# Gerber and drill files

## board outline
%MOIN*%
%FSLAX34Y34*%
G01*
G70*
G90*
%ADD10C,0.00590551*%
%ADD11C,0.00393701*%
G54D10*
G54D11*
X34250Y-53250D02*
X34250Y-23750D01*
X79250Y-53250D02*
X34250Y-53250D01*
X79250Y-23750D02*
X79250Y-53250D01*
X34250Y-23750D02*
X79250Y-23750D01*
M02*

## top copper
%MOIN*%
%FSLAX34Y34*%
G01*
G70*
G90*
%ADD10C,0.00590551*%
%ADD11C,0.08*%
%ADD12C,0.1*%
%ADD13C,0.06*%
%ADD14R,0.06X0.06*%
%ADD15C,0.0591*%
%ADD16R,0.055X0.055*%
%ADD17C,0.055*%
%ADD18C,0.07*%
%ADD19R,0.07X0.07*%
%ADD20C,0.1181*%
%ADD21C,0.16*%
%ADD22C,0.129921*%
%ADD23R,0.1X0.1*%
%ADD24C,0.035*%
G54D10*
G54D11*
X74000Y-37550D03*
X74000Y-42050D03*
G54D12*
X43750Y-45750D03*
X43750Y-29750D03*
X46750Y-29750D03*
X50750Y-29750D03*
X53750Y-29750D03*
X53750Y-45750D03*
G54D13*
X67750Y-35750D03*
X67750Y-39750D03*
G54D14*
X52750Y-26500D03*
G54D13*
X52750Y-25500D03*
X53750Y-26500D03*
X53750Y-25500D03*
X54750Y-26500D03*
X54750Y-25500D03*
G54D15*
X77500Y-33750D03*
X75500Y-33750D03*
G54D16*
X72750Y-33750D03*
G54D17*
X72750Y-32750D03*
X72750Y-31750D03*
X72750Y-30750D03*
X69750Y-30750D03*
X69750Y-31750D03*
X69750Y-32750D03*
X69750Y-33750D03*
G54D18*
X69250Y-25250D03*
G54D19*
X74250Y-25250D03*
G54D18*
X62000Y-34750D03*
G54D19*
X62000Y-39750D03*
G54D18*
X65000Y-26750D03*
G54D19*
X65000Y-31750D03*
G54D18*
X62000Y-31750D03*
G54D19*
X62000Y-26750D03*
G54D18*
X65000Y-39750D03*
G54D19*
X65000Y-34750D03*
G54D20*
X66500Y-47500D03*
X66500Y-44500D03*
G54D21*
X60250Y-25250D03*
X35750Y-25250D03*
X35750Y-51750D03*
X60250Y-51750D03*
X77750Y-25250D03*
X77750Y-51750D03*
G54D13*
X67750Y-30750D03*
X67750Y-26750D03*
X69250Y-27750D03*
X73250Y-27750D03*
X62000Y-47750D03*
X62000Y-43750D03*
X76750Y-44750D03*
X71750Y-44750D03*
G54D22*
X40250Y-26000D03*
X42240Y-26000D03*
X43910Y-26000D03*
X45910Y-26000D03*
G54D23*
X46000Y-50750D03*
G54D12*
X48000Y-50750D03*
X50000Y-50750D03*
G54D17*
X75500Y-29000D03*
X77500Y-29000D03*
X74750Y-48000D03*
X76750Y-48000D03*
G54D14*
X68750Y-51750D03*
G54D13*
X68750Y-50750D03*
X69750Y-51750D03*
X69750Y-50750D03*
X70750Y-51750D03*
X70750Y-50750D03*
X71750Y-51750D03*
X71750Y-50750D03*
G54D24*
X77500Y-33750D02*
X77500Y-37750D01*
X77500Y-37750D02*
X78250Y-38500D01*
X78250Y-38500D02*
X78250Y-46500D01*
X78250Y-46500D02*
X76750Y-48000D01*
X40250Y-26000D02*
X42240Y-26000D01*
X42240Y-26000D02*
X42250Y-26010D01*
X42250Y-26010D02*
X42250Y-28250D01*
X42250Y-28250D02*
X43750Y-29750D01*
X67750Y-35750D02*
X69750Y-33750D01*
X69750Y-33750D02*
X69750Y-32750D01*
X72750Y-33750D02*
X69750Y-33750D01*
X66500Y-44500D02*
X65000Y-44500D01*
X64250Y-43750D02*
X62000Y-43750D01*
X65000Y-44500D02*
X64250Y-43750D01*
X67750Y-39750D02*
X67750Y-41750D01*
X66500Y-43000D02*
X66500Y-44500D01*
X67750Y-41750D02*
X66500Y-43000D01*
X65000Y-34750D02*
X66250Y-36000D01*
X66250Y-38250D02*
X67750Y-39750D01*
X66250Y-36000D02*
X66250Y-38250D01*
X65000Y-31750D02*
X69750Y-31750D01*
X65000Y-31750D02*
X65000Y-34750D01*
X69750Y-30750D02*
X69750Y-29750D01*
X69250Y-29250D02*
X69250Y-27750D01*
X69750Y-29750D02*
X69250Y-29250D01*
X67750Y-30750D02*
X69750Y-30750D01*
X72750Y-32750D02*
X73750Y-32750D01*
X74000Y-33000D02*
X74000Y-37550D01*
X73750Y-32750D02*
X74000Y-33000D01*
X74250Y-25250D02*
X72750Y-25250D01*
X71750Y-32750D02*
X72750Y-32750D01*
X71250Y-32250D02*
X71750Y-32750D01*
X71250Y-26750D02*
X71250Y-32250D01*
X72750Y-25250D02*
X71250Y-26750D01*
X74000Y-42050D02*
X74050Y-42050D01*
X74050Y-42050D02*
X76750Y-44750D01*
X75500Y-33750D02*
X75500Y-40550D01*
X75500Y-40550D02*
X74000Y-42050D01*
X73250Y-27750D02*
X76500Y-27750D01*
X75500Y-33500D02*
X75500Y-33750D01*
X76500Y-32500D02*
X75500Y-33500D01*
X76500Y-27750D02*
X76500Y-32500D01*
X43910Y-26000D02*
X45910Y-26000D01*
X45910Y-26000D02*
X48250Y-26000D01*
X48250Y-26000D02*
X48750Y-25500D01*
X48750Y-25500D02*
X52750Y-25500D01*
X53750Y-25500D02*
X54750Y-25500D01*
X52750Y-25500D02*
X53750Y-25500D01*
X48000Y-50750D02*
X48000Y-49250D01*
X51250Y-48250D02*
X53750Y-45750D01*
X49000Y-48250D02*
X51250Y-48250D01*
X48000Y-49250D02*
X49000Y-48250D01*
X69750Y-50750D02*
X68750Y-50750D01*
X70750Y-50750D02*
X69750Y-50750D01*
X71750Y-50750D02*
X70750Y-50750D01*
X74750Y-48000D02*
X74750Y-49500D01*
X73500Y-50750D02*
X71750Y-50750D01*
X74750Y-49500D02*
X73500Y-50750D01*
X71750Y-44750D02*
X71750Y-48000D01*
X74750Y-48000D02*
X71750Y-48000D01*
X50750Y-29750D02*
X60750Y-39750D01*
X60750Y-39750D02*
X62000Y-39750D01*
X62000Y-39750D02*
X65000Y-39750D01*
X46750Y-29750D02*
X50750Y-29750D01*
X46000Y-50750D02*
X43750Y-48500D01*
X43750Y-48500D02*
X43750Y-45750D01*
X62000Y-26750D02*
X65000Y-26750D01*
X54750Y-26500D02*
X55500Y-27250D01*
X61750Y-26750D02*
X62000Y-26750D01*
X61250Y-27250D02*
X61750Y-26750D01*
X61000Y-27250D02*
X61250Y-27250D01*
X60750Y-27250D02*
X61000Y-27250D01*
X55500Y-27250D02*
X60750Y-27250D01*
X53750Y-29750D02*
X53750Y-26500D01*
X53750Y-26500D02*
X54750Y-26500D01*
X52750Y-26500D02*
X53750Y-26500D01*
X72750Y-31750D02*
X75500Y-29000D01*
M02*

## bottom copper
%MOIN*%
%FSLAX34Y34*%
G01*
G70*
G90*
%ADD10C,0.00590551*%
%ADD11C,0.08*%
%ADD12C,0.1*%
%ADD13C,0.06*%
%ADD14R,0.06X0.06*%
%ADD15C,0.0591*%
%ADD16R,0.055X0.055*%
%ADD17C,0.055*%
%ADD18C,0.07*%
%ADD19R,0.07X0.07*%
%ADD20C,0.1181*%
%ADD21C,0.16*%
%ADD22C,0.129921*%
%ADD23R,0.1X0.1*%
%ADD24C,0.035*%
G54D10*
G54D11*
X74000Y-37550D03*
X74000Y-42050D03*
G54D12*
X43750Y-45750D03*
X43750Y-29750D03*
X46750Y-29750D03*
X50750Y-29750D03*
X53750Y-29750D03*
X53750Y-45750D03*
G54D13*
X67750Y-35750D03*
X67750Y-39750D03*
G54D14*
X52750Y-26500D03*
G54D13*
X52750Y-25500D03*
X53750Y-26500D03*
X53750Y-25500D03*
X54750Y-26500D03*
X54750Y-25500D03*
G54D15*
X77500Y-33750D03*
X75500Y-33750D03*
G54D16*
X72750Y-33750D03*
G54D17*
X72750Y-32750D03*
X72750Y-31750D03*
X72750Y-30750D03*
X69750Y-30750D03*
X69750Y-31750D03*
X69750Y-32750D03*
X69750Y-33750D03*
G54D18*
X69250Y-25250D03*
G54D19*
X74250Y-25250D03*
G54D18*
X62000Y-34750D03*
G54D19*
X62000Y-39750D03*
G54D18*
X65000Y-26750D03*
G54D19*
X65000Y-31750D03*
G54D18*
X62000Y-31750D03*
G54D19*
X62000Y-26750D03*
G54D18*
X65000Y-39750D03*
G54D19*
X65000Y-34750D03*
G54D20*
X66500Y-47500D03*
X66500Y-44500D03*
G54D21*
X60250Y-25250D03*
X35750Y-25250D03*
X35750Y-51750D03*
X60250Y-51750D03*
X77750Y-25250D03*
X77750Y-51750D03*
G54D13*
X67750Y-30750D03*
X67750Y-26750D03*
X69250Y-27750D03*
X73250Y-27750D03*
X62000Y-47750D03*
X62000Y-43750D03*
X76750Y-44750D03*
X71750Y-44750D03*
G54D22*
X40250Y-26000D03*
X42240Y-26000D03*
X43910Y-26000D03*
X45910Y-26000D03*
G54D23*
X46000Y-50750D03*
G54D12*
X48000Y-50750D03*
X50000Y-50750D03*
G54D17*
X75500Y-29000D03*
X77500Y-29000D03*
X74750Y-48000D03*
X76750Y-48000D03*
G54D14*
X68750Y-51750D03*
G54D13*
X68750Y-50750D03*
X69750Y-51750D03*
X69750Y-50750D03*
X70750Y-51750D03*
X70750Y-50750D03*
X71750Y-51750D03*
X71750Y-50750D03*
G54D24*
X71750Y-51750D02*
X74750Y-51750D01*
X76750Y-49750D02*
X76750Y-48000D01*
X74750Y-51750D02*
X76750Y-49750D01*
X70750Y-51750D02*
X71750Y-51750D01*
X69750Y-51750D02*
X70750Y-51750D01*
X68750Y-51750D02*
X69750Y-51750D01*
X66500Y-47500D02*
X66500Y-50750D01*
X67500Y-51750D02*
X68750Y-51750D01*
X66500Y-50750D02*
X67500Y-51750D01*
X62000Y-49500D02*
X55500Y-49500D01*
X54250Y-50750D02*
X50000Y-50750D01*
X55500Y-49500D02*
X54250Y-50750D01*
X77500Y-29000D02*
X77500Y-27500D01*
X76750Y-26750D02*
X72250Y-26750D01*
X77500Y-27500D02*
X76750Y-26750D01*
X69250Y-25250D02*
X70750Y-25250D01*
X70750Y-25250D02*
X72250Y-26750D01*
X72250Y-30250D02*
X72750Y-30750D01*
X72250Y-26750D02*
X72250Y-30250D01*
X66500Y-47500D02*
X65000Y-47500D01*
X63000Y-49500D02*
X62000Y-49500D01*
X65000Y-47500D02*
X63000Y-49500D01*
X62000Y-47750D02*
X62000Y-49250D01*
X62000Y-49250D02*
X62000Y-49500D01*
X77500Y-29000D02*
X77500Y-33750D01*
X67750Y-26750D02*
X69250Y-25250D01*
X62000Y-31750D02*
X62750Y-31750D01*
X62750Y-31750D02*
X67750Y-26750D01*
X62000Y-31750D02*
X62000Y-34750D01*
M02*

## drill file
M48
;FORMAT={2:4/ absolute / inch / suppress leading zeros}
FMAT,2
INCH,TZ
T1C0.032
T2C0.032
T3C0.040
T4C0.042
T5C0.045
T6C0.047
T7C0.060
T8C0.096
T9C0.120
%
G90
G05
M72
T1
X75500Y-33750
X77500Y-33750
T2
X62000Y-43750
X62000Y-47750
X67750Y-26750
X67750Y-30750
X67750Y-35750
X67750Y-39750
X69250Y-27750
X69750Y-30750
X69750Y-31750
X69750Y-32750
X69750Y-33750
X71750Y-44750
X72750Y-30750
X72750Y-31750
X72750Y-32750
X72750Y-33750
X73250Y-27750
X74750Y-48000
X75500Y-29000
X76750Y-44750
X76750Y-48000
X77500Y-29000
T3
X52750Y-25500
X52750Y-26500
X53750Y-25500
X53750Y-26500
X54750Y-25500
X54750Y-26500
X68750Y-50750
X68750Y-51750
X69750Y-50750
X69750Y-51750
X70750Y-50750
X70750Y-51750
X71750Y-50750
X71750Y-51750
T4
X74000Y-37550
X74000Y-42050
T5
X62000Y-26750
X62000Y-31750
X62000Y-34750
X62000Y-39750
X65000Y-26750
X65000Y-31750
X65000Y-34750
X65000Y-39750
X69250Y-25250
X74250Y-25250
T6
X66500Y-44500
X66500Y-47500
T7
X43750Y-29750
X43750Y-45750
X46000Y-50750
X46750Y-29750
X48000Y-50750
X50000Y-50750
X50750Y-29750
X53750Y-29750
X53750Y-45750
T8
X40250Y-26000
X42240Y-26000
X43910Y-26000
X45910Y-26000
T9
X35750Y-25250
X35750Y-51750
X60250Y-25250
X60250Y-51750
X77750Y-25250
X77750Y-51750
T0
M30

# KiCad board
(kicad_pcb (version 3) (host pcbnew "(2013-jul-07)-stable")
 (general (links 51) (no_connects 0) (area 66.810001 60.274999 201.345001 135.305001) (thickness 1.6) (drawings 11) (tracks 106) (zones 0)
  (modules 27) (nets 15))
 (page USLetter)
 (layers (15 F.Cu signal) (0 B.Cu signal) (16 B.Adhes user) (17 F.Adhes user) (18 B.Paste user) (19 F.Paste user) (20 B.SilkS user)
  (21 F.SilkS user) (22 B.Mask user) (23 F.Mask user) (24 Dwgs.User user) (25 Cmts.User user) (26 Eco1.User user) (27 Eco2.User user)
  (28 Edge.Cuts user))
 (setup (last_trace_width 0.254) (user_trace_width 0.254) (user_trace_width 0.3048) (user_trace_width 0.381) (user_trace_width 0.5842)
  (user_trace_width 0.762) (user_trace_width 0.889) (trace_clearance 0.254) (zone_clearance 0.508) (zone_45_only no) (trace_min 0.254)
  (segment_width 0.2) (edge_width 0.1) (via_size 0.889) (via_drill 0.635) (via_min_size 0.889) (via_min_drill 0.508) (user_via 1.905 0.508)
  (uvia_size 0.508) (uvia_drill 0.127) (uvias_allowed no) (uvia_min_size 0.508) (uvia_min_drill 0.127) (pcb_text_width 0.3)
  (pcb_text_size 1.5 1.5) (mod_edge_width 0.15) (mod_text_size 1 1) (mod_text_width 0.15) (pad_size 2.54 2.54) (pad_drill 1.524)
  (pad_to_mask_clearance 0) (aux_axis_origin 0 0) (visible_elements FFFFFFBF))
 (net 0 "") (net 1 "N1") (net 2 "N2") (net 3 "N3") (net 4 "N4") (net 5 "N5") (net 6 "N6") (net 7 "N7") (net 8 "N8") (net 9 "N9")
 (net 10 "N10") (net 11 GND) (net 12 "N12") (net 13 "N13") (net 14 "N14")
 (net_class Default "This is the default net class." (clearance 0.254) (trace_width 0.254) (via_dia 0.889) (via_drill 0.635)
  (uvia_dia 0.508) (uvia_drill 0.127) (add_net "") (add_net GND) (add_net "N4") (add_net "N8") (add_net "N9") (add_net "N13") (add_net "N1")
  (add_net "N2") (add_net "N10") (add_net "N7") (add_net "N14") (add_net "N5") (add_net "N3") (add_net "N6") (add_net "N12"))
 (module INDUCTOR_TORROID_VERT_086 (layer F.Cu) (at 187.96 100.965)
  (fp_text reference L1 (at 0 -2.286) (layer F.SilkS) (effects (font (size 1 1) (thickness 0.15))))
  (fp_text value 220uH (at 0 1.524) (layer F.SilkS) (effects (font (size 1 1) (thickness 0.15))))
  (pad 1 thru_hole circle (at 0 -5.588) (size 2.032 2.032) (drill 1.0668) (layers *.Cu *.Mask F.SilkS) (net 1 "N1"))
  (pad 2 thru_hole circle (at 0 5.842) (size 2.032 2.032) (drill 1.0668) (layers *.Cu *.Mask F.SilkS) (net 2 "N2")))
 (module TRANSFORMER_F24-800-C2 (layer F.Cu) (at 123.825 75.565)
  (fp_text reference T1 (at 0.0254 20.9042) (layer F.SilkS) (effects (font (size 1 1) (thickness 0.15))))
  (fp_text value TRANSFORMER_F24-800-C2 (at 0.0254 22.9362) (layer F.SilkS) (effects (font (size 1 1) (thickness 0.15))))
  (pad 1 thru_hole circle (at -12.7 40.64) (size 2.54 2.54) (drill 1.524) (layers *.Cu *.Mask F.SilkS) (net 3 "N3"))
  (pad 5 thru_hole circle (at -12.7 0) (size 2.54 2.54) (drill 1.524) (layers *.Cu *.Mask F.SilkS) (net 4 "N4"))
  (pad 6 thru_hole circle (at -5.08 0) (size 2.54 2.54) (drill 1.524) (layers *.Cu *.Mask F.SilkS) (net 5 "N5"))
  (pad 7 thru_hole circle (at 5.08 0) (size 2.54 2.54) (drill 1.524) (layers *.Cu *.Mask F.SilkS) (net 5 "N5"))
  (pad 8 thru_hole circle (at 12.7 0) (size 2.54 2.54) (drill 1.524) (layers *.Cu *.Mask F.SilkS) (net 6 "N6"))
  (pad 4 thru_hole circle (at 12.7 40.64) (size 2.54 2.54) (drill 1.524) (layers *.Cu *.Mask F.SilkS) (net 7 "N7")))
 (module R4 (layer F.Cu) (at 172.085 95.885 270) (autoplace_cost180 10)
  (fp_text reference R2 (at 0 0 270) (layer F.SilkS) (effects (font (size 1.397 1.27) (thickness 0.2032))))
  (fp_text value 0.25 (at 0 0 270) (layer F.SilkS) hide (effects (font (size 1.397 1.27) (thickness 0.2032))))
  (pad 1 thru_hole circle (at -5.08 0 270) (size 1.524 1.524) (drill 0.8128) (layers *.Cu *.Mask F.SilkS) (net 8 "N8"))
  (pad 2 thru_hole circle (at 5.08 0 270) (size 1.524 1.524) (drill 0.8128) (layers *.Cu *.Mask F.SilkS) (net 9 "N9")))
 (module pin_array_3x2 (layer F.Cu) (at 136.525 66.04)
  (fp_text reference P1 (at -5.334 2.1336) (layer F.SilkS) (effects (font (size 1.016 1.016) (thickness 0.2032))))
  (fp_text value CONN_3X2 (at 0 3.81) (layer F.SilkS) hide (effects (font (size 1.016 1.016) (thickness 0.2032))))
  (pad 1 thru_hole rect (at -2.54 1.27) (size 1.524 1.524) (drill 1.016) (layers *.Cu *.Mask F.SilkS) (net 6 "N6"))
  (pad 2 thru_hole circle (at -2.54 -1.27) (size 1.524 1.524) (drill 1.016) (layers *.Cu *.Mask F.SilkS) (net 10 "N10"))
  (pad 3 thru_hole circle (at 0 1.27) (size 1.524 1.524) (drill 1.016) (layers *.Cu *.Mask F.SilkS) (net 6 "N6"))
  (pad 4 thru_hole circle (at 0 -1.27) (size 1.524 1.524) (drill 1.016) (layers *.Cu *.Mask F.SilkS) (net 10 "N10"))
  (pad 5 thru_hole circle (at 2.54 1.27) (size 1.524 1.524) (drill 1.016) (layers *.Cu *.Mask F.SilkS) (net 6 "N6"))
  (pad 6 thru_hole circle (at 2.54 -1.27) (size 1.524 1.524) (drill 1.016) (layers *.Cu *.Mask F.SilkS) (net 10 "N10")))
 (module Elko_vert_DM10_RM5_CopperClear (layer F.Cu) (at 194.31 85.725)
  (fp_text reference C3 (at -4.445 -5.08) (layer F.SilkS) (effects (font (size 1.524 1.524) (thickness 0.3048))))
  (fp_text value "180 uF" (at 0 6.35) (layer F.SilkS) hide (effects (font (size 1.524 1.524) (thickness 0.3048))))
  (pad 2 thru_hole circle (at 2.54 0) (size 1.50114 1.50114) (drill 0.8001) (layers *.Cu *.Mask F.SilkS) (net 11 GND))
  (pad 1 thru_hole circle (at -2.54 0) (size 1.50114 1.50114) (drill 0.8001) (layers *.Cu *.Mask F.SilkS) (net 2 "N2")))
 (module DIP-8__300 (layer F.Cu) (at 180.975 81.915 90)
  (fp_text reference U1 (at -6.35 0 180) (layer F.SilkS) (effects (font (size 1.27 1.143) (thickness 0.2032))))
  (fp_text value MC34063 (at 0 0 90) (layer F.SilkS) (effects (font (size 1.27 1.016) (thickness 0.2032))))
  (pad 1 thru_hole rect (at -3.81 3.81 90) (size 1.397 1.397) (drill 0.8128) (layers *.Cu *.Mask F.SilkS) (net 8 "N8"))
  (pad 2 thru_hole circle (at -1.27 3.81 90) (size 1.397 1.397) (drill 0.8128) (layers *.Cu *.Mask F.SilkS) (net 1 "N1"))
  (pad 3 thru_hole circle (at 1.27 3.81 90) (size 1.397 1.397) (drill 0.8128) (layers *.Cu *.Mask F.SilkS) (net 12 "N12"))
  (pad 4 thru_hole circle (at 3.81 3.81 90) (size 1.397 1.397) (drill 0.8128) (layers *.Cu *.Mask F.SilkS) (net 11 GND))
  (pad 5 thru_hole circle (at 3.81 -3.81 90) (size 1.397 1.397) (drill 0.8128) (layers *.Cu *.Mask F.SilkS) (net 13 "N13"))
  (pad 6 thru_hole circle (at 1.27 -3.81 90) (size 1.397 1.397) (drill 0.8128) (layers *.Cu *.Mask F.SilkS) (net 9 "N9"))
  (pad 7 thru_hole circle (at -1.27 -3.81 90) (size 1.397 1.397) (drill 0.8128) (layers *.Cu *.Mask F.SilkS) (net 8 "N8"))
  (pad 8 thru_hole circle (at -3.81 -3.81 90) (size 1.397 1.397) (drill 0.8128) (layers *.Cu *.Mask F.SilkS) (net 8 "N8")))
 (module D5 (layer F.Cu) (at 182.245 64.135)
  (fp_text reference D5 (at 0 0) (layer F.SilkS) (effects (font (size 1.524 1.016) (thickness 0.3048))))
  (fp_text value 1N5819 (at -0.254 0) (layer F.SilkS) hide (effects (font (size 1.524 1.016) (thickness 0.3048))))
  (pad 1 thru_hole circle (at -6.35 0) (size 1.778 1.778) (drill 1.143) (layers *.Cu *.Mask F.SilkS) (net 11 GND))
  (pad 2 thru_hole rect (at 6.35 0) (size 1.778 1.778) (drill 1.143) (layers *.Cu *.Mask F.SilkS) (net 1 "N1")))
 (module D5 (layer F.Cu) (at 157.48 94.615 270)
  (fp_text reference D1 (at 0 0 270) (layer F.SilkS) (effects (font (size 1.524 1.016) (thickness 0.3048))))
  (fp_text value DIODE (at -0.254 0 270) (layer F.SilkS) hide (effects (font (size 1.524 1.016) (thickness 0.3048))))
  (pad 1 thru_hole circle (at -6.35 0 270) (size 1.778 1.778) (drill 1.143) (layers *.Cu *.Mask F.SilkS) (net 11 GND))
  (pad 2 thru_hole rect (at 6.35 0 270) (size 1.778 1.778) (drill 1.143) (layers *.Cu *.Mask F.SilkS) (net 5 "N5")))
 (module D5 (layer F.Cu) (at 165.1 74.295 270)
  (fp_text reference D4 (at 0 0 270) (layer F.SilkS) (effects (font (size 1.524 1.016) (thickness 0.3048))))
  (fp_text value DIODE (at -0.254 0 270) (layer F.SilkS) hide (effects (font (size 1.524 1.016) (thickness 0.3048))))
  (pad 1 thru_hole circle (at -6.35 0 270) (size 1.778 1.778) (drill 1.143) (layers *.Cu *.Mask F.SilkS) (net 6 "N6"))
  (pad 2 thru_hole rect (at 6.35 0 270) (size 1.778 1.778) (drill 1.143) (layers *.Cu *.Mask F.SilkS) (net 9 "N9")))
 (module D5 (layer F.Cu) (at 157.48 74.295 90)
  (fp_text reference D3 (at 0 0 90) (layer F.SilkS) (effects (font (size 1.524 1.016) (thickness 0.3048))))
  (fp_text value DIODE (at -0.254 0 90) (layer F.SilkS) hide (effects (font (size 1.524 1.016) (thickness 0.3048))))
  (pad 1 thru_hole circle (at -6.35 0 90) (size 1.778 1.778) (drill 1.143) (layers *.Cu *.Mask F.SilkS) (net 11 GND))
  (pad 2 thru_hole rect (at 6.35 0 90) (size 1.778 1.778) (drill 1.143) (layers *.Cu *.Mask F.SilkS) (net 6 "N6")))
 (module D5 (layer F.Cu) (at 165.1 94.615 90)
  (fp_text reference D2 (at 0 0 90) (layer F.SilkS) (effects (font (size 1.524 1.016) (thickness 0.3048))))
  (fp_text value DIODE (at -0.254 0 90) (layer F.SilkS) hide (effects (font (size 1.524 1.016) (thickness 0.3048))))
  (pad 1 thru_hole circle (at -6.35 0 90) (size 1.778 1.778) (drill 1.143) (layers *.Cu *.Mask F.SilkS) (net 5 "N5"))
  (pad 2 thru_hole rect (at 6.35 0 90) (size 1.778 1.778) (drill 1.143) (layers *.Cu *.Mask F.SilkS) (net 9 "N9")))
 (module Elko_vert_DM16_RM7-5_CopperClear (layer F.Cu) (at 168.91 116.84 270)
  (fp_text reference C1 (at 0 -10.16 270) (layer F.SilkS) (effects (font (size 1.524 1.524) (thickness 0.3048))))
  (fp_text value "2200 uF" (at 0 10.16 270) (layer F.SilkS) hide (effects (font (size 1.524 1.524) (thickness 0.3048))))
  (pad 2 thru_hole circle (at 3.81 0 270) (size 2.99974 2.99974) (drill 1.19888) (layers *.Cu *.Mask F.SilkS) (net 11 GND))
  (pad 1 thru_hole circle (at -3.81 0 270) (size 2.99974 2.99974) (drill 1.19888) (layers *.Cu *.Mask F.SilkS) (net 9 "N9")))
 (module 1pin (layer F.Cu) (at 153.035 64.135)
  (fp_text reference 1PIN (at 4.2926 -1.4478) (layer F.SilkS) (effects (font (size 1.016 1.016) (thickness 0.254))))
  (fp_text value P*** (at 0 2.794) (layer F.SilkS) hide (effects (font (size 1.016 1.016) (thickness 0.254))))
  (pad 1 thru_hole circle (at 0 0) (size 4.064 4.064) (drill 3.048) (layers *.Cu *.Mask F.SilkS)))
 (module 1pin (layer F.Cu) (at 90.805 64.135)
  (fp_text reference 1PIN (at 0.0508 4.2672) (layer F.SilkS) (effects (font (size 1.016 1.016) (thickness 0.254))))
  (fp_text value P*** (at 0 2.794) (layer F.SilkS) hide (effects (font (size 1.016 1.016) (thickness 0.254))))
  (pad 1 thru_hole circle (at 0 0) (size 4.064 4.064) (drill 3.048) (layers *.Cu *.Mask F.SilkS)))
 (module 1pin (layer F.Cu) (at 90.805 131.445)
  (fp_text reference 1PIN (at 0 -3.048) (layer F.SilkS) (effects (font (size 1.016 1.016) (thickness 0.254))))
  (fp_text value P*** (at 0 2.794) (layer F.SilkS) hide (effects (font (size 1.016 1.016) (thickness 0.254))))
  (pad 1 thru_hole circle (at 0 0) (size 4.064 4.064) (drill 3.048) (layers *.Cu *.Mask F.SilkS)))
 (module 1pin (layer F.Cu) (at 153.035 131.445)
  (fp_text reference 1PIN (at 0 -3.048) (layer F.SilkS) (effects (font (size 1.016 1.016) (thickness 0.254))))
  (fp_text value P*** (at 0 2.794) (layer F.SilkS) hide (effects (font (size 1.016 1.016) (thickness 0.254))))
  (pad 1 thru_hole circle (at 0 0) (size 4.064 4.064) (drill 3.048) (layers *.Cu *.Mask F.SilkS)))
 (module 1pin (layer F.Cu) (at 197.485 64.135)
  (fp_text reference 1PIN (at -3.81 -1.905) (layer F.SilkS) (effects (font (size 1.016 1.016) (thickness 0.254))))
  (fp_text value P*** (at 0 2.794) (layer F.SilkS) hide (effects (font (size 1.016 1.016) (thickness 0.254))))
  (pad 1 thru_hole circle (at 0 0) (size 4.064 4.064) (drill 3.048) (layers *.Cu *.Mask F.SilkS)))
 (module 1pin (layer F.Cu) (at 197.485 131.445)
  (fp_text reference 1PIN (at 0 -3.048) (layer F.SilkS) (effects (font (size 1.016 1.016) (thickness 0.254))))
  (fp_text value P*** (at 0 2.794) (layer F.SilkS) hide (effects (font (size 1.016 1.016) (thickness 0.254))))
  (pad 1 thru_hole circle (at 0 0) (size 4.064 4.064) (drill 3.048) (layers *.Cu *.Mask F.SilkS)))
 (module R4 (layer F.Cu) (at 172.085 73.025 90) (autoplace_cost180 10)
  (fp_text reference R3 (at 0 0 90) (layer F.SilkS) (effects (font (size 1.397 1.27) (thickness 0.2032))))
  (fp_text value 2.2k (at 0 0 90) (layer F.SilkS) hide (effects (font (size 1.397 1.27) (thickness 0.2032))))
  (pad 1 thru_hole circle (at -5.08 0 90) (size 1.524 1.524) (drill 0.8128) (layers *.Cu *.Mask F.SilkS) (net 13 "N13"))
  (pad 2 thru_hole circle (at 5.08 0 90) (size 1.524 1.524) (drill 0.8128) (layers *.Cu *.Mask F.SilkS) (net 11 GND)))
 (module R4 (layer F.Cu) (at 180.975 70.485) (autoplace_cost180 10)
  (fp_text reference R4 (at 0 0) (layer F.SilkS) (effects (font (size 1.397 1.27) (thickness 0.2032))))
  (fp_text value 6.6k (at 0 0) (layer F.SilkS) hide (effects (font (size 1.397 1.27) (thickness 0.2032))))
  (pad 1 thru_hole circle (at -5.08 0) (size 1.524 1.524) (drill 0.8128) (layers *.Cu *.Mask F.SilkS) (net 13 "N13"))
  (pad 2 thru_hole circle (at 5.08 0) (size 1.524 1.524) (drill 0.8128) (layers *.Cu *.Mask F.SilkS) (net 2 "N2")))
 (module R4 (layer F.Cu) (at 157.48 116.205 90) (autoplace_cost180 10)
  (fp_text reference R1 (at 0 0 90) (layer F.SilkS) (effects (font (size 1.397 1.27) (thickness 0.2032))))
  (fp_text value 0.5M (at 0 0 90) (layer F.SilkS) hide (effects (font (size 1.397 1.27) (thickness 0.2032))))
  (pad 1 thru_hole circle (at -5.08 0 90) (size 1.524 1.524) (drill 0.8128) (layers *.Cu *.Mask F.SilkS) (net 11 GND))
  (pad 2 thru_hole circle (at 5.08 0 90) (size 1.524 1.524) (drill 0.8128) (layers *.Cu *.Mask F.SilkS) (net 9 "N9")))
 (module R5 (layer F.Cu) (at 188.595 113.665 180) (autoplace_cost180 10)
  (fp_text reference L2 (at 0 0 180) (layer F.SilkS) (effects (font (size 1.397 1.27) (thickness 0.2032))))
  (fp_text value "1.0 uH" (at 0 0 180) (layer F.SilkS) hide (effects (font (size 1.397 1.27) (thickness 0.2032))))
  (pad 1 thru_hole circle (at -6.35 0 180) (size 1.524 1.524) (drill 0.8128) (layers *.Cu *.Mask F.SilkS) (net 2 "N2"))
  (pad 2 thru_hole circle (at 6.35 0 180) (size 1.524 1.524) (drill 0.8128) (layers *.Cu *.Mask F.SilkS) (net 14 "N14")))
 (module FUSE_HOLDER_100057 (layer F.Cu) (at 109.855 66.04)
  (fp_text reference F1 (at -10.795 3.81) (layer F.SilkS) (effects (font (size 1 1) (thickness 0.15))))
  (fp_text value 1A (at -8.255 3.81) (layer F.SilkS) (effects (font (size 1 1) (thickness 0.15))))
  (pad 1 thru_hole circle (at -7.62 0) (size 3.3 3.3) (drill 2.44) (layers *.Cu *.Mask F.SilkS) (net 4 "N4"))
  (pad 1 thru_hole circle (at -2.5654 0) (size 3.3 3.3) (drill 2.44) (layers *.Cu *.Mask F.SilkS) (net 4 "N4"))
  (pad 2 thru_hole circle (at 1.6764 0) (size 3.3 3.3) (drill 2.44) (layers *.Cu *.Mask F.SilkS) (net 10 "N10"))
  (pad 2 thru_hole circle (at 6.7564 0) (size 3.3 3.3) (drill 2.44) (layers *.Cu *.Mask F.SilkS) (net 10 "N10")))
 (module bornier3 (layer F.Cu) (at 121.92 128.905)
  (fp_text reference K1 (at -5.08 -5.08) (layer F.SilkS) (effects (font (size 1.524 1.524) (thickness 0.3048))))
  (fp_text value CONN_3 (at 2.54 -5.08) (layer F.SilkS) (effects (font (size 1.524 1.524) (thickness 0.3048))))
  (pad 1 thru_hole rect (at -5.08 0) (size 2.54 2.54) (drill 1.524) (layers *.Cu *.Mask F.SilkS) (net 3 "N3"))
  (pad 2 thru_hole circle (at 0 0) (size 2.54 2.54) (drill 1.524) (layers *.Cu *.Mask F.SilkS) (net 7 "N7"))
  (pad 3 thru_hole circle (at 5.08 0) (size 2.54 2.54) (drill 1.524) (layers *.Cu *.Mask F.SilkS) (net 11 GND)))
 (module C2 (layer F.Cu) (at 194.31 73.66)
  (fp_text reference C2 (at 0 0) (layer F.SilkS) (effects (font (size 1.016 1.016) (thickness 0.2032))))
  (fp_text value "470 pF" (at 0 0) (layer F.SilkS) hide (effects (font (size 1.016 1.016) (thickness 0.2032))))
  (pad 1 thru_hole circle (at -2.54 0) (size 1.397 1.397) (drill 0.8128) (layers *.Cu *.Mask F.SilkS) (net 12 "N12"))
  (pad 2 thru_hole circle (at 2.54 0) (size 1.397 1.397) (drill 0.8128) (layers *.Cu *.Mask F.SilkS) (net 11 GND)))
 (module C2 (layer F.Cu) (at 192.405 121.92)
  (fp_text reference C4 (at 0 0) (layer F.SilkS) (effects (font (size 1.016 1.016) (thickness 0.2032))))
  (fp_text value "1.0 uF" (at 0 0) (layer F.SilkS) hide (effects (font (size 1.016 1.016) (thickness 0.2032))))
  (pad 1 thru_hole circle (at -2.54 0) (size 1.397 1.397) (drill 0.8128) (layers *.Cu *.Mask F.SilkS) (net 14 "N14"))
  (pad 2 thru_hole circle (at 2.54 0) (size 1.397 1.397) (drill 0.8128) (layers *.Cu *.Mask F.SilkS) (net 11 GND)))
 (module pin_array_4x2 (layer F.Cu) (at 178.435 130.175)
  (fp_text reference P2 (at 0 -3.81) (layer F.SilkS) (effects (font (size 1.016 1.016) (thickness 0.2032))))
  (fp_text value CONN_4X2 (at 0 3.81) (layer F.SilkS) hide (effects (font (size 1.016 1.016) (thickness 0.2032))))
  (pad 1 thru_hole rect (at -3.81 1.27) (size 1.524 1.524) (drill 1.016) (layers *.Cu *.Mask F.SilkS) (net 11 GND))
  (pad 2 thru_hole circle (at -3.81 -1.27) (size 1.524 1.524) (drill 1.016) (layers *.Cu *.Mask F.SilkS) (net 14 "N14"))
  (pad 3 thru_hole circle (at -1.27 1.27) (size 1.524 1.524) (drill 1.016) (layers *.Cu *.Mask F.SilkS) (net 11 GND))
  (pad 4 thru_hole circle (at -1.27 -1.27) (size 1.524 1.524) (drill 1.016) (layers *.Cu *.Mask F.SilkS) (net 14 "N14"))
  (pad 5 thru_hole circle (at 1.27 1.27) (size 1.524 1.524) (drill 1.016) (layers *.Cu *.Mask F.SilkS) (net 11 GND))
  (pad 6 thru_hole circle (at 1.27 -1.27) (size 1.524 1.524) (drill 1.016) (layers *.Cu *.Mask F.SilkS) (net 14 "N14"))
  (pad 7 thru_hole circle (at 3.81 1.27) (size 1.524 1.524) (drill 1.016) (layers *.Cu *.Mask F.SilkS) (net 11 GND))
  (pad 8 thru_hole circle (at 3.81 -1.27) (size 1.524 1.524) (drill 1.016) (layers *.Cu *.Mask F.SilkS) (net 14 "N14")))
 (gr_line (start 86.995 135.255) (end 86.995 60.325) (angle 90) (layer Edge.Cuts) (width 0.1))
 (gr_line (start 201.295 135.255) (end 86.995 135.255) (angle 90) (layer Edge.Cuts) (width 0.1))
 (gr_line (start 201.295 60.325) (end 201.295 135.255) (angle 90) (layer Edge.Cuts) (width 0.1))
 (gr_line (start 86.995 60.325) (end 201.295 60.325) (angle 90) (layer Edge.Cuts) (width 0.1))
 (segment (start 182.245 131.445) (end 189.865 131.445) (width 0.889) (layer B.Cu) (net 11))
 (segment (start 194.945 126.365) (end 194.945 121.92) (width 0.889) (layer B.Cu) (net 11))
 (segment (start 189.865 131.445) (end 194.945 126.365) (width 0.889) (layer B.Cu) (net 11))
 (segment (start 179.705 131.445) (end 182.245 131.445) (width 0.889) (layer B.Cu) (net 11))
 (segment (start 177.165 131.445) (end 179.705 131.445) (width 0.889) (layer B.Cu) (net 11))
 (segment (start 174.625 131.445) (end 177.165 131.445) (width 0.889) (layer B.Cu) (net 11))
 (segment (start 168.91 120.65) (end 168.91 128.905) (width 0.889) (layer B.Cu) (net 11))
 (segment (start 171.45 131.445) (end 174.625 131.445) (width 0.889) (layer B.Cu) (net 11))
 (segment (start 168.91 128.905) (end 171.45 131.445) (width 0.889) (layer B.Cu) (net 11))
 (segment (start 157.48 125.73) (end 140.97 125.73) (width 0.889) (layer B.Cu) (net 11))
 (segment (start 137.795 128.905) (end 127 128.905) (width 0.889) (layer B.Cu) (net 11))
 (segment (start 140.97 125.73) (end 137.795 128.905) (width 0.889) (layer B.Cu) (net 11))
 (segment (start 196.85 73.66) (end 196.85 69.85) (width 0.889) (layer B.Cu) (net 11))
 (segment (start 194.945 67.945) (end 183.515 67.945) (width 0.889) (layer B.Cu) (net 11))
 (segment (start 196.85 69.85) (end 194.945 67.945) (width 0.889) (layer B.Cu) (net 11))
 (segment (start 175.895 64.135) (end 179.705 64.135) (width 0.889) (layer B.Cu) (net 11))
 (segment (start 179.705 64.135) (end 183.515 67.945) (width 0.889) (layer B.Cu) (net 11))
 (segment (start 183.515 76.835) (end 184.785 78.105) (width 0.889) (layer B.Cu) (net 11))
 (segment (start 183.515 67.945) (end 183.515 76.835) (width 0.889) (layer B.Cu) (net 11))
 (segment (start 168.91 120.65) (end 165.1 120.65) (width 0.889) (layer B.Cu) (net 11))
 (segment (start 160.02 125.73) (end 157.48 125.73) (width 0.889) (layer B.Cu) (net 11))
 (segment (start 165.1 120.65) (end 160.02 125.73) (width 0.889) (layer B.Cu) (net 11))
 (segment (start 157.48 121.285) (end 157.48 125.095) (width 0.889) (layer B.Cu) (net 11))
 (segment (start 157.48 125.095) (end 157.48 125.73) (width 0.889) (layer B.Cu) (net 11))
 (segment (start 196.85 85.725) (end 196.85 95.885) (width 0.889) (layer F.Cu) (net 11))
 (segment (start 196.85 95.885) (end 198.755 97.79) (width 0.889) (layer F.Cu) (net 11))
 (segment (start 198.755 97.79) (end 198.755 118.11) (width 0.889) (layer F.Cu) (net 11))
 (segment (start 198.755 118.11) (end 194.945 121.92) (width 0.889) (layer F.Cu) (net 11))
 (segment (start 196.85 73.66) (end 196.85 85.725) (width 0.889) (layer B.Cu) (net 11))
 (segment (start 172.085 67.945) (end 175.895 64.135) (width 0.889) (layer B.Cu) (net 11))
 (segment (start 157.48 80.645) (end 159.385 80.645) (width 0.889) (layer B.Cu) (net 11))
 (segment (start 159.385 80.645) (end 172.085 67.945) (width 0.889) (layer B.Cu) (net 11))
 (segment (start 157.48 80.645) (end 157.48 88.265) (width 0.889) (layer B.Cu) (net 11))
 (segment (start 102.235 66.04) (end 107.2896 66.04) (width 0.889) (layer F.Cu) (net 4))
 (segment (start 107.2896 66.04) (end 107.315 66.0654) (width 0.889) (layer F.Cu) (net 4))
 (segment (start 107.315 66.0654) (end 107.315 71.755) (width 0.889) (layer F.Cu) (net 4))
 (segment (start 107.315 71.755) (end 111.125 75.565) (width 0.889) (layer F.Cu) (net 4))
 (segment (start 172.085 90.805) (end 177.165 85.725) (width 0.889) (layer F.Cu) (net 8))
 (segment (start 177.165 85.725) (end 177.165 83.185) (width 0.889) (layer F.Cu) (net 8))
 (segment (start 184.785 85.725) (end 177.165 85.725) (width 0.889) (layer F.Cu) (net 8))
 (segment (start 168.91 113.03) (end 165.1 113.03) (width 0.889) (layer F.Cu) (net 9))
 (segment (start 163.195 111.125) (end 157.48 111.125) (width 0.889) (layer F.Cu) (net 9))
 (segment (start 165.1 113.03) (end 163.195 111.125) (width 0.889) (layer F.Cu) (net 9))
 (segment (start 172.085 100.965) (end 172.085 106.045) (width 0.889) (layer F.Cu) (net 9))
 (segment (start 168.91 109.22) (end 168.91 113.03) (width 0.889) (layer F.Cu) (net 9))
 (segment (start 172.085 106.045) (end 168.91 109.22) (width 0.889) (layer F.Cu) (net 9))
 (segment (start 165.1 88.265) (end 168.275 91.44) (width 0.889) (layer F.Cu) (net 9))
 (segment (start 168.275 97.155) (end 172.085 100.965) (width 0.889) (layer F.Cu) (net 9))
 (segment (start 168.275 91.44) (end 168.275 97.155) (width 0.889) (layer F.Cu) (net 9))
 (segment (start 165.1 80.645) (end 177.165 80.645) (width 0.889) (layer F.Cu) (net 9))
 (segment (start 165.1 80.645) (end 165.1 88.265) (width 0.889) (layer F.Cu) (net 9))
 (segment (start 177.165 78.105) (end 177.165 75.565) (width 0.889) (layer F.Cu) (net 13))
 (segment (start 175.895 74.295) (end 175.895 70.485) (width 0.889) (layer F.Cu) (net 13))
 (segment (start 177.165 75.565) (end 175.895 74.295) (width 0.889) (layer F.Cu) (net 13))
 (segment (start 172.085 78.105) (end 177.165 78.105) (width 0.889) (layer F.Cu) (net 13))
 (segment (start 184.785 83.185) (end 187.325 83.185) (width 0.889) (layer F.Cu) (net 1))
 (segment (start 187.96 83.82) (end 187.96 95.377) (width 0.889) (layer F.Cu) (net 1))
 (segment (start 187.325 83.185) (end 187.96 83.82) (width 0.889) (layer F.Cu) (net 1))
 (segment (start 188.595 64.135) (end 184.785 64.135) (width 0.889) (layer F.Cu) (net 1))
 (segment (start 182.245 83.185) (end 184.785 83.185) (width 0.889) (layer F.Cu) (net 1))
 (segment (start 180.975 81.915) (end 182.245 83.185) (width 0.889) (layer F.Cu) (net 1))
 (segment (start 180.975 67.945) (end 180.975 81.915) (width 0.889) (layer F.Cu) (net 1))
 (segment (start 184.785 64.135) (end 180.975 67.945) (width 0.889) (layer F.Cu) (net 1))
 (segment (start 187.96 106.807) (end 188.087 106.807) (width 0.889) (layer F.Cu) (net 2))
 (segment (start 188.087 106.807) (end 194.945 113.665) (width 0.889) (layer F.Cu) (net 2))
 (segment (start 191.77 85.725) (end 191.77 102.997) (width 0.889) (layer F.Cu) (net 2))
 (segment (start 191.77 102.997) (end 187.96 106.807) (width 0.889) (layer F.Cu) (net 2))
 (segment (start 186.055 70.485) (end 194.31 70.485) (width 0.889) (layer F.Cu) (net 2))
 (segment (start 191.77 85.09) (end 191.77 85.725) (width 0.889) (layer F.Cu) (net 2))
 (segment (start 194.31 82.55) (end 191.77 85.09) (width 0.889) (layer F.Cu) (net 2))
 (segment (start 194.31 70.485) (end 194.31 82.55) (width 0.889) (layer F.Cu) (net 2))
 (segment (start 111.5314 66.04) (end 116.6114 66.04) (width 0.889) (layer F.Cu) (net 10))
 (segment (start 116.6114 66.04) (end 122.555 66.04) (width 0.889) (layer F.Cu) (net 10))
 (segment (start 122.555 66.04) (end 123.825 64.77) (width 0.889) (layer F.Cu) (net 10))
 (segment (start 123.825 64.77) (end 133.985 64.77) (width 0.889) (layer F.Cu) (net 10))
 (segment (start 136.525 64.77) (end 139.065 64.77) (width 0.889) (layer F.Cu) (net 10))
 (segment (start 133.985 64.77) (end 136.525 64.77) (width 0.889) (layer F.Cu) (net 10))
 (segment (start 121.92 128.905) (end 121.92 125.095) (width 0.889) (layer F.Cu) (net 7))
 (segment (start 130.175 122.555) (end 136.525 116.205) (width 0.889) (layer F.Cu) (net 7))
 (segment (start 124.46 122.555) (end 130.175 122.555) (width 0.889) (layer F.Cu) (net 7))
 (segment (start 121.92 125.095) (end 124.46 122.555) (width 0.889) (layer F.Cu) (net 7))
 (segment (start 177.165 128.905) (end 174.625 128.905) (width 0.889) (layer F.Cu) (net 14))
 (segment (start 179.705 128.905) (end 177.165 128.905) (width 0.889) (layer F.Cu) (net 14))
 (segment (start 182.245 128.905) (end 179.705 128.905) (width 0.889) (layer F.Cu) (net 14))
 (segment (start 189.865 121.92) (end 189.865 125.73) (width 0.889) (layer F.Cu) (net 14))
 (segment (start 186.69 128.905) (end 182.245 128.905) (width 0.889) (layer F.Cu) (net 14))
 (segment (start 189.865 125.73) (end 186.69 128.905) (width 0.889) (layer F.Cu) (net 14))
 (segment (start 182.245 113.665) (end 182.245 121.92) (width 0.889) (layer F.Cu) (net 14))
 (segment (start 189.865 121.92) (end 182.245 121.92) (width 0.889) (layer F.Cu) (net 14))
 (segment (start 128.905 75.565) (end 154.305 100.965) (width 0.889) (layer F.Cu) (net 5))
 (segment (start 154.305 100.965) (end 157.48 100.965) (width 0.889) (layer F.Cu) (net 5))
 (segment (start 157.48 100.965) (end 165.1 100.965) (width 0.889) (layer F.Cu) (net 5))
 (segment (start 118.745 75.565) (end 128.905 75.565) (width 0.889) (layer F.Cu) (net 5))
 (segment (start 116.84 128.905) (end 111.125 123.19) (width 0.889) (layer F.Cu) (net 3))
 (segment (start 111.125 123.19) (end 111.125 116.205) (width 0.889) (layer F.Cu) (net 3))
 (segment (start 157.48 67.945) (end 165.1 67.945) (width 0.889) (layer F.Cu) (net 6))
 (segment (start 139.065 67.31) (end 140.97 69.215) (width 0.889) (layer F.Cu) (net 6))
 (segment (start 156.845 67.945) (end 157.48 67.945) (width 0.889) (layer F.Cu) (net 6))
 (segment (start 155.575 69.215) (end 156.845 67.945) (width 0.889) (layer F.Cu) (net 6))
 (segment (start 154.94 69.215) (end 155.575 69.215) (width 0.889) (layer F.Cu) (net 6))
 (segment (start 154.305 69.215) (end 154.94 69.215) (width 0.889) (layer F.Cu) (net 6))
 (segment (start 140.97 69.215) (end 154.305 69.215) (width 0.889) (layer F.Cu) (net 6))
 (segment (start 136.525 75.565) (end 136.525 67.31) (width 0.889) (layer F.Cu) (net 6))
 (segment (start 136.525 67.31) (end 139.065 67.31) (width 0.889) (layer F.Cu) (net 6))
 (segment (start 133.985 67.31) (end 136.525 67.31) (width 0.889) (layer F.Cu) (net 6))
 (segment (start 184.785 80.645) (end 191.77 73.66) (width 0.889) (layer F.Cu) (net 12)))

